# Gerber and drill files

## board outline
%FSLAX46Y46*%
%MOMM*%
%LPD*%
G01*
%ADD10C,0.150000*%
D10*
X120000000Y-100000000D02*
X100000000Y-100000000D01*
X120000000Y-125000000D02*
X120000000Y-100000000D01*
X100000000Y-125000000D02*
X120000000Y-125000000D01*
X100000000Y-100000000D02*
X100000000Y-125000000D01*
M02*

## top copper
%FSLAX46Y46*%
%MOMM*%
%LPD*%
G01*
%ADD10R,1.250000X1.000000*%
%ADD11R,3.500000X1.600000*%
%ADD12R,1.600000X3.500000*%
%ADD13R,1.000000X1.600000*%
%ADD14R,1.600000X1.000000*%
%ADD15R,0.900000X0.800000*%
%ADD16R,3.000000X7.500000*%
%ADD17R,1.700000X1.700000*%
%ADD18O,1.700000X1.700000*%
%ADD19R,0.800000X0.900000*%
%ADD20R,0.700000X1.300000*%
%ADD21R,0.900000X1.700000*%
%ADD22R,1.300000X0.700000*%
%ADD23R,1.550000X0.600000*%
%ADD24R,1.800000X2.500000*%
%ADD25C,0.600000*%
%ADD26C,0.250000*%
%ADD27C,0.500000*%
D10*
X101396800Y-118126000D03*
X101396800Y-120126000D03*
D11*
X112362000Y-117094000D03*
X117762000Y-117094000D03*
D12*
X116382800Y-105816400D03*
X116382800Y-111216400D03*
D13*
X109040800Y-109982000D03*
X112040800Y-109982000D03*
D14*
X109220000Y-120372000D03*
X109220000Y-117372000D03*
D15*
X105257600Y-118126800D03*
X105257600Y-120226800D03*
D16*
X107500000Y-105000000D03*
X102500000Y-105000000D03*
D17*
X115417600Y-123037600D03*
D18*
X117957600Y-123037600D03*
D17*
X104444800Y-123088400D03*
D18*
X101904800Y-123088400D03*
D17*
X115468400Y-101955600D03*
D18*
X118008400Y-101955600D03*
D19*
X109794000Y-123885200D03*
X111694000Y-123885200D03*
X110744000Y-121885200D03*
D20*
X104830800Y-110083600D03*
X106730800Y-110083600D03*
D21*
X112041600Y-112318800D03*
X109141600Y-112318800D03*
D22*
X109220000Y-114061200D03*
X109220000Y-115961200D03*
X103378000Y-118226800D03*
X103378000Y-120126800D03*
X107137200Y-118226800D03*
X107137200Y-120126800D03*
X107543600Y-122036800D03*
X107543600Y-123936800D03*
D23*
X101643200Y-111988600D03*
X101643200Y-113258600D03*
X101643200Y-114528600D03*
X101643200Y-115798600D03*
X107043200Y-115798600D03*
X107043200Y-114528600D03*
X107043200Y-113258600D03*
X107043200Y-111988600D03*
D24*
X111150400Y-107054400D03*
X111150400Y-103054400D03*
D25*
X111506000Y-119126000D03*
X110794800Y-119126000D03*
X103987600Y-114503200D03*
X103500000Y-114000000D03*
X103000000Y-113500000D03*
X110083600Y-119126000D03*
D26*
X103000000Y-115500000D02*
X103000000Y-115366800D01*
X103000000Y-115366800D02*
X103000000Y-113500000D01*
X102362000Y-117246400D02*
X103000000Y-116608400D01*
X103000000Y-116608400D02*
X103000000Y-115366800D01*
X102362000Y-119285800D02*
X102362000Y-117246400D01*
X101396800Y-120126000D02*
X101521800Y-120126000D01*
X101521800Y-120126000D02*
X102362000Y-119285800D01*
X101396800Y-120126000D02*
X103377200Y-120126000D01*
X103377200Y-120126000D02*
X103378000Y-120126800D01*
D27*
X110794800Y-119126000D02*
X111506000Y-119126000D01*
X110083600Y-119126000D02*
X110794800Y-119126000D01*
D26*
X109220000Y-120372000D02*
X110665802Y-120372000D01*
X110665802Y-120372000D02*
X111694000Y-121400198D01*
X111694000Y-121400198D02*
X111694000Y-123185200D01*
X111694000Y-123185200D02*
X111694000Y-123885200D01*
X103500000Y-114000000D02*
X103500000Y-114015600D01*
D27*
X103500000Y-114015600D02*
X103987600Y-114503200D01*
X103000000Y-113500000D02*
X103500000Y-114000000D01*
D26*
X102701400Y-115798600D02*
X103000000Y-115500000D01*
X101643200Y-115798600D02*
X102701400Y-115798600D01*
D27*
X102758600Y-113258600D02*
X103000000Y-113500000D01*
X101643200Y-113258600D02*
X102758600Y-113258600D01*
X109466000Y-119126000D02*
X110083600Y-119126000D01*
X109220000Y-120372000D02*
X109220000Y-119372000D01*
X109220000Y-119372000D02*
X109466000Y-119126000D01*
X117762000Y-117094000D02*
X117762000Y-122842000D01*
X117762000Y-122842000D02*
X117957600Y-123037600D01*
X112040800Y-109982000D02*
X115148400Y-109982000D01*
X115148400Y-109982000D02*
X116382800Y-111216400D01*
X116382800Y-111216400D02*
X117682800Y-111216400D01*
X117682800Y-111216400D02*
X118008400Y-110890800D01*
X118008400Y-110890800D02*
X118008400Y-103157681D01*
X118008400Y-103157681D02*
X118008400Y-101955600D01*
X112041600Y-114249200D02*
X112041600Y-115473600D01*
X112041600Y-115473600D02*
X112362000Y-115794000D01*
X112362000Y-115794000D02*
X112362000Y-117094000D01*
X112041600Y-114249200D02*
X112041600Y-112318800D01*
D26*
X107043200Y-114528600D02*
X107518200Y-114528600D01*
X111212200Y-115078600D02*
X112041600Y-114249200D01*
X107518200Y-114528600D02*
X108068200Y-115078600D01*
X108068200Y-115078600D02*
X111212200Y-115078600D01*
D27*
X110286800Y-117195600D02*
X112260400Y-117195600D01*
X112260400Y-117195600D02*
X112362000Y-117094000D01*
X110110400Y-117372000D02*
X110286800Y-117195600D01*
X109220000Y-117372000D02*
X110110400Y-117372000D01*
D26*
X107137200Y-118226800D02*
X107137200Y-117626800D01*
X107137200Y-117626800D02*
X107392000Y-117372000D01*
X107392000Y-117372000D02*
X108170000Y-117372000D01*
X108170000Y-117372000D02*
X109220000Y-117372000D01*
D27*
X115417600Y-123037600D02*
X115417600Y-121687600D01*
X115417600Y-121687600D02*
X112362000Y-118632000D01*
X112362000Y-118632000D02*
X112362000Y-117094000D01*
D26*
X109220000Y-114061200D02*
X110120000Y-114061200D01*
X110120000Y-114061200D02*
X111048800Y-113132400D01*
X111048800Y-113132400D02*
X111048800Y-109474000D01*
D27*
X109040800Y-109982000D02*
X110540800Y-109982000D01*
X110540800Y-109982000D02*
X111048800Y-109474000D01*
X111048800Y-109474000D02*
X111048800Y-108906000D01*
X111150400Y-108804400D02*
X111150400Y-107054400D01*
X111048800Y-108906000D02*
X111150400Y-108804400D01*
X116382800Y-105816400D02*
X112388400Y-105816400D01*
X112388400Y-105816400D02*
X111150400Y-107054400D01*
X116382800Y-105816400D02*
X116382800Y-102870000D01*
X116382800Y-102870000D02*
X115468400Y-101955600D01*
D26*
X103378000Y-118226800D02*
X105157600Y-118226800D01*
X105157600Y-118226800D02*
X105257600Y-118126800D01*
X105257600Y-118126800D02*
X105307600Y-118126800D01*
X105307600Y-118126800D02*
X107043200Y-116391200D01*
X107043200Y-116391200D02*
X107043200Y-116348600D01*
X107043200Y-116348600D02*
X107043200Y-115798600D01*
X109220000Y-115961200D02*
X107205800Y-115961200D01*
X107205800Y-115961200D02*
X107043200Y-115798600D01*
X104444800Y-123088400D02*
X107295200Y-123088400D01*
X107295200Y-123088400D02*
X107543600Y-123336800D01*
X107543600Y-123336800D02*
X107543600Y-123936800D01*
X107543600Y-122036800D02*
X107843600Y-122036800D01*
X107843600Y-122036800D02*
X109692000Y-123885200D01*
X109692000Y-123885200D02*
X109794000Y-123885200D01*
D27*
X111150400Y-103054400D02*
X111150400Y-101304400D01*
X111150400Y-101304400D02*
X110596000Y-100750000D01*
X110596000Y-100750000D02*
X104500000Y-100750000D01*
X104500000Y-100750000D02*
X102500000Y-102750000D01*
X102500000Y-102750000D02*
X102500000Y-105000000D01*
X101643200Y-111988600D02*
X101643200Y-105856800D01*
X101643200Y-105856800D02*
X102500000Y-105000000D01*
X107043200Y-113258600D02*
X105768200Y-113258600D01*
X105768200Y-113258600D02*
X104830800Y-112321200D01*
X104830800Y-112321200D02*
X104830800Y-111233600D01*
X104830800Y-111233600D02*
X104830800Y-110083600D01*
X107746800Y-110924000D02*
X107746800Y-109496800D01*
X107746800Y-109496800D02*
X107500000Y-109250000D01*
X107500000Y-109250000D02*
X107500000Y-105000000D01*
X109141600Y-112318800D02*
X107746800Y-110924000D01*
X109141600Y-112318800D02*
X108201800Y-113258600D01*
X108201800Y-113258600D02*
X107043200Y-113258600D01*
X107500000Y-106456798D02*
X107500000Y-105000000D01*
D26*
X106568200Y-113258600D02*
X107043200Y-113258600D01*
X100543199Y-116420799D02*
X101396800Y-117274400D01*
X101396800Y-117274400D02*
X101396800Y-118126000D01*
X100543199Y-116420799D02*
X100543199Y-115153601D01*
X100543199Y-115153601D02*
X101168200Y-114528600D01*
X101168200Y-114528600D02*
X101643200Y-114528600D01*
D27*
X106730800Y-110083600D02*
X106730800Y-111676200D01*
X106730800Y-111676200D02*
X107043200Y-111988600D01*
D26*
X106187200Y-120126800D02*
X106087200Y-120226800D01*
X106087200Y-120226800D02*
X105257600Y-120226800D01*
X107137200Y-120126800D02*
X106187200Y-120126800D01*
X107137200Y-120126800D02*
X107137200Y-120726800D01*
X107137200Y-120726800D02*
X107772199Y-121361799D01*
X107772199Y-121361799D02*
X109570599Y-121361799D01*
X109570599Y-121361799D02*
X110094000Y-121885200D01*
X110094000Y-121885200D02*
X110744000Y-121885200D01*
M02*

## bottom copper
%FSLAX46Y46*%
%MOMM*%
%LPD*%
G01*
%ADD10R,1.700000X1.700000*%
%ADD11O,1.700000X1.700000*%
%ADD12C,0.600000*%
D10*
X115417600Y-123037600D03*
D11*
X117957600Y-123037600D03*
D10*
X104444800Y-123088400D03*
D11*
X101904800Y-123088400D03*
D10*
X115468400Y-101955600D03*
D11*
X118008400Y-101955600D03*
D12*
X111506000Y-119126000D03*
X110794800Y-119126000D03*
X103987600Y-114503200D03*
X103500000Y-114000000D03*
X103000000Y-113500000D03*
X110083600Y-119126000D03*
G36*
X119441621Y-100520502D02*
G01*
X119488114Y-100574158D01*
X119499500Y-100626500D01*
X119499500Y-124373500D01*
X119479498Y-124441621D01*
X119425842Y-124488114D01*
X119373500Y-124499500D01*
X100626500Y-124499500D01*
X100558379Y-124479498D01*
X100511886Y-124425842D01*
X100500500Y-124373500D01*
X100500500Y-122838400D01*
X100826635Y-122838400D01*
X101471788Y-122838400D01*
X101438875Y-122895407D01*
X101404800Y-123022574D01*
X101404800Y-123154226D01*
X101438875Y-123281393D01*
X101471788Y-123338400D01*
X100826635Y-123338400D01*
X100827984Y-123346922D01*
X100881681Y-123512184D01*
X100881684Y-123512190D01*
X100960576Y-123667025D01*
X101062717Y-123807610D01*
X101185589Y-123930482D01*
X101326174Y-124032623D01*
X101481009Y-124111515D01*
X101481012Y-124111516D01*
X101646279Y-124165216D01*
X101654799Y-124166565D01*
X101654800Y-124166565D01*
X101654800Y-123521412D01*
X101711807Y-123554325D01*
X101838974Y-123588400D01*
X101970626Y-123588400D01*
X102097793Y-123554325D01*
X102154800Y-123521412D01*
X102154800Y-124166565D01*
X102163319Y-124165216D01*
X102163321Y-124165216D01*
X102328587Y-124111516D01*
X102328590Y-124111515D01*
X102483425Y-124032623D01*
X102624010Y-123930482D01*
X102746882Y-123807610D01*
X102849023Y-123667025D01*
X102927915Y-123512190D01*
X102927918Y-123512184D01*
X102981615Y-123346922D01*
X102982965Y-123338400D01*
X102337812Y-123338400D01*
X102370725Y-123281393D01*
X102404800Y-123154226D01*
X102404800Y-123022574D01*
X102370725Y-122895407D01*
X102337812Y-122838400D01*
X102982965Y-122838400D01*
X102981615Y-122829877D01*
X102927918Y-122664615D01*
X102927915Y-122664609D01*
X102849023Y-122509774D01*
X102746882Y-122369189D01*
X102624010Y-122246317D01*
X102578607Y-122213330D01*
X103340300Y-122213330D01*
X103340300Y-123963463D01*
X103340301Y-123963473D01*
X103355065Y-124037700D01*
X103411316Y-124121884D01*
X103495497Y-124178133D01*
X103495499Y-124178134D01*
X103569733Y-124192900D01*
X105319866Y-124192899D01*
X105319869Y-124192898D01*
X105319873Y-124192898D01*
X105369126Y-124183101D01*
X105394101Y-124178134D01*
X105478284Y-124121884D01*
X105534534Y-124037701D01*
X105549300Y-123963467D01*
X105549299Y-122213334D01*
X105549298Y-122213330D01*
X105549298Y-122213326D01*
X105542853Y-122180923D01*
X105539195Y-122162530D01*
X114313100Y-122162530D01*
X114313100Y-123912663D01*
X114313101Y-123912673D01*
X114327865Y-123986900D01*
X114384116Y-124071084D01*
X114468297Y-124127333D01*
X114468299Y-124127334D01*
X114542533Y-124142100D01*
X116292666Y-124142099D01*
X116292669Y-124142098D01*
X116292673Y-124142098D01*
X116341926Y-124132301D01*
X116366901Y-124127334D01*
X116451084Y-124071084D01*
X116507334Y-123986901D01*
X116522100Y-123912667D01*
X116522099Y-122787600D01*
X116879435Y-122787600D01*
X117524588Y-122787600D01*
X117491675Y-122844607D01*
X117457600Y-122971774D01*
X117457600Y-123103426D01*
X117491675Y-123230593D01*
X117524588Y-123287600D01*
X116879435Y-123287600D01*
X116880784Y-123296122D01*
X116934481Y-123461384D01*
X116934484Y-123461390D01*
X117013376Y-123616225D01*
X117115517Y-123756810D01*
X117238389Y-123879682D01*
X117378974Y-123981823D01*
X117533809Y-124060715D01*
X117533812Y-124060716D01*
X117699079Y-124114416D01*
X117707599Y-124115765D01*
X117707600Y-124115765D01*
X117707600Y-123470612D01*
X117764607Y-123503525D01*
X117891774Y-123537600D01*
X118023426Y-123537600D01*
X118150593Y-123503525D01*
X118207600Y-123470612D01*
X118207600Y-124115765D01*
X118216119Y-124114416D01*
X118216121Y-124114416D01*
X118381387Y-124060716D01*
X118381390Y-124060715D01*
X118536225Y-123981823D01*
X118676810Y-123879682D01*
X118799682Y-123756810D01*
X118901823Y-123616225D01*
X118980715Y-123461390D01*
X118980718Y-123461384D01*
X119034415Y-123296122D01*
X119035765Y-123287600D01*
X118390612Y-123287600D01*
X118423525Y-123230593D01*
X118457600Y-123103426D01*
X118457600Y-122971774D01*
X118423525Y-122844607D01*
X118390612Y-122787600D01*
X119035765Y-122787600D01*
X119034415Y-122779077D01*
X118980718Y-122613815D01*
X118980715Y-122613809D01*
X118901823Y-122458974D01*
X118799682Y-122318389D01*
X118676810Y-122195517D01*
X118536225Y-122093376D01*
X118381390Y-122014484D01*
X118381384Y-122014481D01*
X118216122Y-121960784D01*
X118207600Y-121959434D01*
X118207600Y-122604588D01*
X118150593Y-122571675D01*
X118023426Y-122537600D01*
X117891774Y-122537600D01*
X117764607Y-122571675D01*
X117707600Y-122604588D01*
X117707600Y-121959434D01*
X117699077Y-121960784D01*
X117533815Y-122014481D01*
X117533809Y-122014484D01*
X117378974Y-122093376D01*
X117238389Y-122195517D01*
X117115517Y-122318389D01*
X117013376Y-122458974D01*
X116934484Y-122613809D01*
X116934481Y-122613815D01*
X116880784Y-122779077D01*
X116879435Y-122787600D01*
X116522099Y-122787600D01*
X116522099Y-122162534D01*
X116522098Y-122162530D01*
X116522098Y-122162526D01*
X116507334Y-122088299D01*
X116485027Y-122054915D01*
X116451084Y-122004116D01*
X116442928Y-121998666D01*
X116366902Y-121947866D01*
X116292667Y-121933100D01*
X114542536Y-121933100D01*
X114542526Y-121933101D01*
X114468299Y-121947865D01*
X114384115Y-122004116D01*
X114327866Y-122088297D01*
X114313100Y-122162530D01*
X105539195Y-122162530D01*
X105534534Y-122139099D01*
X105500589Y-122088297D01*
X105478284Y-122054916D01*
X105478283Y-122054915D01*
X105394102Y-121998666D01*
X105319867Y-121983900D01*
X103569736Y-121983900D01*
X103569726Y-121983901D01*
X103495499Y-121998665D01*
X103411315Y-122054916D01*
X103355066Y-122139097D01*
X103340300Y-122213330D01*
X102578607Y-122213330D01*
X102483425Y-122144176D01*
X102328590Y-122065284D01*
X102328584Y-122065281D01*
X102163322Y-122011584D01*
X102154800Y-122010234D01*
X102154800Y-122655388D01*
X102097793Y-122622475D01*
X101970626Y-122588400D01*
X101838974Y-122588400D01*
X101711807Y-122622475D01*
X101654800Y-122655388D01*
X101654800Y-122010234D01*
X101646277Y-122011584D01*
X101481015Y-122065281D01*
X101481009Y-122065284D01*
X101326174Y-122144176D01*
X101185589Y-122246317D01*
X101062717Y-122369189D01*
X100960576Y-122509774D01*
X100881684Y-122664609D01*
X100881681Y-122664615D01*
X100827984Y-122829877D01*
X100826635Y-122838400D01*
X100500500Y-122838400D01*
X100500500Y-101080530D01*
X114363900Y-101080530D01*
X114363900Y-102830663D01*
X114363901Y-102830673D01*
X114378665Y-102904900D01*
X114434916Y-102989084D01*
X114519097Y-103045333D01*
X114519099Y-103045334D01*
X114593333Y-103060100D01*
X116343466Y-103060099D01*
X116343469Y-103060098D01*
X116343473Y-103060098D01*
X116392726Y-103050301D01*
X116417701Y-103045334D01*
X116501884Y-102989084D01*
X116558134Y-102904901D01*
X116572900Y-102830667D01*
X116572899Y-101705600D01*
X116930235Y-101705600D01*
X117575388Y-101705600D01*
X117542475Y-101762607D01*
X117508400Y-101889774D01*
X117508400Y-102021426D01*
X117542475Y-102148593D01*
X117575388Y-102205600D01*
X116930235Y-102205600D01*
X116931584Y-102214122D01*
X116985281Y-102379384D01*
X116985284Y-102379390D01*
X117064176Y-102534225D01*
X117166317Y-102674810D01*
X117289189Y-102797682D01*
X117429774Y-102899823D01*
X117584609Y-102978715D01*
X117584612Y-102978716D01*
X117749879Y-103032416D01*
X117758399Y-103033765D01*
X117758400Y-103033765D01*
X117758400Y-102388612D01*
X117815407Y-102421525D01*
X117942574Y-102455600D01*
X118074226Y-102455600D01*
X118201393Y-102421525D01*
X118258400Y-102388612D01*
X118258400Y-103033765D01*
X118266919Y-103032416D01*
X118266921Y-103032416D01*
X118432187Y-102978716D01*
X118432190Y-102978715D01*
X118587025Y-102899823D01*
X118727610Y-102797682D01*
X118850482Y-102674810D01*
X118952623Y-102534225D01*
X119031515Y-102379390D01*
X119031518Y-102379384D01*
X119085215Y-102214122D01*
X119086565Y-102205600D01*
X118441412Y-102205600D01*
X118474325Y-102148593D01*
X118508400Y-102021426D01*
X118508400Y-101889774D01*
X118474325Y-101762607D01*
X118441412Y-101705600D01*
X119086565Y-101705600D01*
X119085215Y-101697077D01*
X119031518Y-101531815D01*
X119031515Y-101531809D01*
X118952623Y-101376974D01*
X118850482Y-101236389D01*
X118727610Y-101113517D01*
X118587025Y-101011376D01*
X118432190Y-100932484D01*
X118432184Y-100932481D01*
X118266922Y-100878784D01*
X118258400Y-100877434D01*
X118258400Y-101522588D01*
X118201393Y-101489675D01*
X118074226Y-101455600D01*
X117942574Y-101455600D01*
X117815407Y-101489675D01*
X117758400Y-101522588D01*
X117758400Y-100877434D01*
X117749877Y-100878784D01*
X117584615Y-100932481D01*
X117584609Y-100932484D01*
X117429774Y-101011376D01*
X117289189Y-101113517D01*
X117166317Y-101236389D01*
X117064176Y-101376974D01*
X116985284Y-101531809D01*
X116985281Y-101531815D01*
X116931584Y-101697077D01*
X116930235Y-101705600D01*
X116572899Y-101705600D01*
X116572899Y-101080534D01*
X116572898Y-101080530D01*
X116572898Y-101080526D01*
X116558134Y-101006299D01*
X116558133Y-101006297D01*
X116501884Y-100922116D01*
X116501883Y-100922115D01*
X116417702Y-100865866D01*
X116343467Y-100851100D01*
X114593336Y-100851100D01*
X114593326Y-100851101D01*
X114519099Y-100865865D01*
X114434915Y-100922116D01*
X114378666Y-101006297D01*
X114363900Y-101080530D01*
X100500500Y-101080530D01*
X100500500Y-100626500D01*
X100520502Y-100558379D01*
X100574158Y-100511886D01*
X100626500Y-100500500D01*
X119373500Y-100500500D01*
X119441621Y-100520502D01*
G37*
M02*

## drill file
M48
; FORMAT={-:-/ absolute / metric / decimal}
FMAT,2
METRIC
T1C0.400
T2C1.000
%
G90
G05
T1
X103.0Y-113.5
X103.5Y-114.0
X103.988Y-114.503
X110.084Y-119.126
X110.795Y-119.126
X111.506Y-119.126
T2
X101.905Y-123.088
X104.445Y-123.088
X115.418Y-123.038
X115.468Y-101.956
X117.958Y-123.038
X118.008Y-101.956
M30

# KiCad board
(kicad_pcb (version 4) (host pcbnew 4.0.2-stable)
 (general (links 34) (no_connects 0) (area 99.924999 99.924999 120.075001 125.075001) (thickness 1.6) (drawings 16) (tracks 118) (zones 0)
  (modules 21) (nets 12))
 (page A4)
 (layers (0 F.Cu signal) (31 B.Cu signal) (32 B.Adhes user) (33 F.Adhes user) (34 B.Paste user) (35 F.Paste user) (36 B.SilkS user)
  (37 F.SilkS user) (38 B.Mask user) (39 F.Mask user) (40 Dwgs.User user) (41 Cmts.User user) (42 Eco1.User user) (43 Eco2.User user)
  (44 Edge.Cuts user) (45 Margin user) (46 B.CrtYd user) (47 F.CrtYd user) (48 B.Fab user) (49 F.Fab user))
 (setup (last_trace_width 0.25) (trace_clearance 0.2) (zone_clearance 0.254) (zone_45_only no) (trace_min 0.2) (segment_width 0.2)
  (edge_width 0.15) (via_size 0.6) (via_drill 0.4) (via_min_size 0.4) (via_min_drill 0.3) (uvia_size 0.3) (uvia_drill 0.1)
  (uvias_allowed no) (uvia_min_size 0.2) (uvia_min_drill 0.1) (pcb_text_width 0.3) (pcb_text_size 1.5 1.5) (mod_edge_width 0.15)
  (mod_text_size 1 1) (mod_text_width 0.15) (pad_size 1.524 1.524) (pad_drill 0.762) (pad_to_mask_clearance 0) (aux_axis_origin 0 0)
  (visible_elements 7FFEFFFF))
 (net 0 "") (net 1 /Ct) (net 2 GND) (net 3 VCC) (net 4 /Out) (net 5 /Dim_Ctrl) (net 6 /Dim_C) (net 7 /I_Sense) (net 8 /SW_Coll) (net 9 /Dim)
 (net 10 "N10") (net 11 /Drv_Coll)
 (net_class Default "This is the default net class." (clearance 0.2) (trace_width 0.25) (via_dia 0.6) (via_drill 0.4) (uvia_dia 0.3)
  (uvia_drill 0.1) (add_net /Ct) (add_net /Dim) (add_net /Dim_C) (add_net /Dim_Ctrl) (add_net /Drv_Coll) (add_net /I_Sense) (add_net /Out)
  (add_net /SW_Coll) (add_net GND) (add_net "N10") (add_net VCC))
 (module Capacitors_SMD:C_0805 (layer F.Cu) (at 101.3968 119.126 270)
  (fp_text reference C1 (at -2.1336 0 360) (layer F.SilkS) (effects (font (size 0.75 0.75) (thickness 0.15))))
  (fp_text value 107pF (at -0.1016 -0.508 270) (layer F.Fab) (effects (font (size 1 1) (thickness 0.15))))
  (pad 1 smd rect (at -1 0 270) (size 1 1.25) (layers F.Cu F.Paste F.Mask) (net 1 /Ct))
  (pad 2 smd rect (at 1 0 270) (size 1 1.25) (layers F.Cu F.Paste F.Mask) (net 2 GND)))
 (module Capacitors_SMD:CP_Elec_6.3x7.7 (layer F.Cu) (at 115.062 117.094)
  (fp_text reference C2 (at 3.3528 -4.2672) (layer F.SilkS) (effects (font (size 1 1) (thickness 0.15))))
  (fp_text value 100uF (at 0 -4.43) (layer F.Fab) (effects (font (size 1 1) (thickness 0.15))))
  (pad 1 smd rect (at -2.7 0 180) (size 3.5 1.6) (layers F.Cu F.Paste F.Mask) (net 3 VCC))
  (pad 2 smd rect (at 2.7 0 180) (size 3.5 1.6) (layers F.Cu F.Paste F.Mask) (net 2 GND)))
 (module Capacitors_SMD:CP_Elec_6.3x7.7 (layer F.Cu) (at 116.3828 108.5164 270)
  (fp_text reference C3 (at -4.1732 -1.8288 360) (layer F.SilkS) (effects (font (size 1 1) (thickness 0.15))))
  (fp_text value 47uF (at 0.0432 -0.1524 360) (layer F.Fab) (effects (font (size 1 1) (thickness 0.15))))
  (pad 1 smd rect (at -2.7 0 90) (size 3.5 1.6) (layers F.Cu F.Paste F.Mask) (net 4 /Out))
  (pad 2 smd rect (at 2.7 0 90) (size 3.5 1.6) (layers F.Cu F.Paste F.Mask) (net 2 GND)))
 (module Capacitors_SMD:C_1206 (layer F.Cu) (at 110.5408 109.982)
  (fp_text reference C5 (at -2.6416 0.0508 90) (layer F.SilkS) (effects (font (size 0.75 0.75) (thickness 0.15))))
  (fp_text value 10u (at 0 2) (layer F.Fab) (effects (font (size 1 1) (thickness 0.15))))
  (pad 1 smd rect (at -1.5 0) (size 1 1.6) (layers F.Cu F.Paste F.Mask) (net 4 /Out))
  (pad 2 smd rect (at 1.5 0) (size 1 1.6) (layers F.Cu F.Paste F.Mask) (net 2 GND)))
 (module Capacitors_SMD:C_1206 (layer F.Cu) (at 109.22 118.872 90)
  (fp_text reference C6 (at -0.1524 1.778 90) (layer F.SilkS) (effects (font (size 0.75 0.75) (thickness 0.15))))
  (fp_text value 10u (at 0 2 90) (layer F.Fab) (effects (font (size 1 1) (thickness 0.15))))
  (pad 1 smd rect (at -1.5 0 90) (size 1 1.6) (layers F.Cu F.Paste F.Mask) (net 2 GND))
  (pad 2 smd rect (at 1.5 0 90) (size 1 1.6) (layers F.Cu F.Paste F.Mask) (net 3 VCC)))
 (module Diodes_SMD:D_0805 (layer F.Cu) (at 105.2576 119.1768 270)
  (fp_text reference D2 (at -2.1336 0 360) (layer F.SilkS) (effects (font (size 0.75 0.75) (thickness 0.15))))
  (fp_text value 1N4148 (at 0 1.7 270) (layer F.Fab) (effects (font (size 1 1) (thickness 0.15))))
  (pad 1 smd rect (at -1.05 0 270) (size 0.8 0.9) (layers F.Cu F.Paste F.Mask) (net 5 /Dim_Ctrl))
  (pad 2 smd rect (at 1.05 0 270) (size 0.8 0.9) (layers F.Cu F.Paste F.Mask) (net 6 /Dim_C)))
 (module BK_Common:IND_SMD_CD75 (layer F.Cu) (at 105 105 180)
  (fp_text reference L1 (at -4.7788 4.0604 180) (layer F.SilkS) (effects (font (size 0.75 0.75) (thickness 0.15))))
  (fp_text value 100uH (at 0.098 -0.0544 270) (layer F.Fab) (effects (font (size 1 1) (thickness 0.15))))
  (pad 1 smd rect (at -2.5 0 180) (size 3 7.5) (layers F.Cu F.Paste F.Mask) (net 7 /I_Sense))
  (pad 2 smd rect (at 2.5 0 180) (size 3 7.5) (layers F.Cu F.Paste F.Mask) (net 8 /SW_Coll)))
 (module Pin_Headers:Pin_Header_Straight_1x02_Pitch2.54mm (layer F.Cu) (at 115.4176 123.0376 90)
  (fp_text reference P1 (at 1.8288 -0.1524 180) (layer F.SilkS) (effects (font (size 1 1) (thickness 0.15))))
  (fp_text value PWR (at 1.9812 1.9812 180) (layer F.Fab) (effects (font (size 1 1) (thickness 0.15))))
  (pad 1 thru_hole rect (at 0 0 90) (size 1.7 1.7) (drill 1) (layers *.Cu *.Mask) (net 3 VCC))
  (pad 2 thru_hole oval (at 0 2.54 90) (size 1.7 1.7) (drill 1) (layers *.Cu *.Mask) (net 2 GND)))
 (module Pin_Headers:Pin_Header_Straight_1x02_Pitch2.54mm (layer F.Cu) (at 104.4448 123.0884 270)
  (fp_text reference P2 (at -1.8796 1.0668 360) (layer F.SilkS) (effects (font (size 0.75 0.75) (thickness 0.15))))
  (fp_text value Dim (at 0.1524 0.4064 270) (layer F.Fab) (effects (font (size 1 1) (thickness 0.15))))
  (pad 1 thru_hole rect (at 0 0 270) (size 1.7 1.7) (drill 1) (layers *.Cu *.Mask) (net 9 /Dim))
  (pad 2 thru_hole oval (at 0 2.54 270) (size 1.7 1.7) (drill 1) (layers *.Cu *.Mask) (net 2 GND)))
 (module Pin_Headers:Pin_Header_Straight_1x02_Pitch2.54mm (layer F.Cu) (at 115.4684 101.9556 90)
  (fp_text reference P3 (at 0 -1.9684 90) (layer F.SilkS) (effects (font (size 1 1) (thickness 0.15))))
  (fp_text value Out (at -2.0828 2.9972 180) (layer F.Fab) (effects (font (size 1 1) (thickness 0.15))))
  (pad 1 thru_hole rect (at 0 0 90) (size 1.7 1.7) (drill 1) (layers *.Cu *.Mask) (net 4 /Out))
  (pad 2 thru_hole oval (at 0 2.54 90) (size 1.7 1.7) (drill 1) (layers *.Cu *.Mask) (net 2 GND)))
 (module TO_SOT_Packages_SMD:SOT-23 (layer F.Cu) (at 110.744 122.8852 90)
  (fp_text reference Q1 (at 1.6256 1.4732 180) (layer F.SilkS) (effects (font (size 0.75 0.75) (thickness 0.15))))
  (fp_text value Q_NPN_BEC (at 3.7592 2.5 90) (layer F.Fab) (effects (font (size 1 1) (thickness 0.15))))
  (pad 1 smd rect (at -1 -0.95 90) (size 0.9 0.8) (layers F.Cu F.Paste F.Mask) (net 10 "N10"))
  (pad 2 smd rect (at -1 0.95 90) (size 0.9 0.8) (layers F.Cu F.Paste F.Mask) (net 2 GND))
  (pad 3 smd rect (at 1 0 90) (size 0.9 0.8) (layers F.Cu F.Paste F.Mask) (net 6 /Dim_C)))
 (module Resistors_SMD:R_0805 (layer F.Cu) (at 105.7808 110.0836)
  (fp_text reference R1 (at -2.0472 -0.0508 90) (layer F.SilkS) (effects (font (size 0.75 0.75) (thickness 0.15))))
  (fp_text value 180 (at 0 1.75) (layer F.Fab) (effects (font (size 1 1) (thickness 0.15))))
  (pad 1 smd rect (at -0.95 0) (size 0.7 1.3) (layers F.Cu F.Paste F.Mask) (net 7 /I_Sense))
  (pad 2 smd rect (at 0.95 0) (size 0.7 1.3) (layers F.Cu F.Paste F.Mask) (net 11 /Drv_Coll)))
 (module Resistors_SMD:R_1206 (layer F.Cu) (at 110.5916 112.3188 180)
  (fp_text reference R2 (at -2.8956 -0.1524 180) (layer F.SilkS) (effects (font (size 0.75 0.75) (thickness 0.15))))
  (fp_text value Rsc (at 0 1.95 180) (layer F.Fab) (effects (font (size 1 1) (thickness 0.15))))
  (pad 1 smd rect (at -1.45 0 180) (size 0.9 1.7) (layers F.Cu F.Paste F.Mask) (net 3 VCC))
  (pad 2 smd rect (at 1.45 0 180) (size 0.9 1.7) (layers F.Cu F.Paste F.Mask) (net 7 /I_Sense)))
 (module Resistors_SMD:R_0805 (layer F.Cu) (at 109.22 115.0112 270)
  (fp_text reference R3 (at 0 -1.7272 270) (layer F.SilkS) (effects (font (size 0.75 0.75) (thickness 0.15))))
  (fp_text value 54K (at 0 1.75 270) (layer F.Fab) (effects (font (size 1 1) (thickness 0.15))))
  (pad 1 smd rect (at -0.95 0 270) (size 0.7 1.3) (layers F.Cu F.Paste F.Mask) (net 4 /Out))
  (pad 2 smd rect (at 0.95 0 270) (size 0.7 1.3) (layers F.Cu F.Paste F.Mask) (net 5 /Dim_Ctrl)))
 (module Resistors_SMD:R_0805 (layer F.Cu) (at 103.378 119.1768 270)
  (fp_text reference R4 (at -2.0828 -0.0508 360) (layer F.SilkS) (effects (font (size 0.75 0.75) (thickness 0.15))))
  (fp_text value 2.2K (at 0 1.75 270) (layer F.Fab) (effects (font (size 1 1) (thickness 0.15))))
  (pad 1 smd rect (at -0.95 0 270) (size 0.7 1.3) (layers F.Cu F.Paste F.Mask) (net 5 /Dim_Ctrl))
  (pad 2 smd rect (at 0.95 0 270) (size 0.7 1.3) (layers F.Cu F.Paste F.Mask) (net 2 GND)))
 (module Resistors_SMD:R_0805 (layer F.Cu) (at 107.1372 119.1768 270)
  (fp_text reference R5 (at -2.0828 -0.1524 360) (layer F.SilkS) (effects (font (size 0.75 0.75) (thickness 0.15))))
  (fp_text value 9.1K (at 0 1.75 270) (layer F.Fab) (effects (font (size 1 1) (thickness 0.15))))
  (pad 1 smd rect (at -0.95 0 270) (size 0.7 1.3) (layers F.Cu F.Paste F.Mask) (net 3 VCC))
  (pad 2 smd rect (at 0.95 0 270) (size 0.7 1.3) (layers F.Cu F.Paste F.Mask) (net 6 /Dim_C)))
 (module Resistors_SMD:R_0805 (layer F.Cu) (at 107.5436 122.9868 270)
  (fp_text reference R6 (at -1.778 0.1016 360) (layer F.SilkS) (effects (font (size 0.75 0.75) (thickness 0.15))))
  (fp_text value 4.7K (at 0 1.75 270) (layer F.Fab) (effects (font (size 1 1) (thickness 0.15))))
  (pad 1 smd rect (at -0.95 0 270) (size 0.7 1.3) (layers F.Cu F.Paste F.Mask) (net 10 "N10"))
  (pad 2 smd rect (at 0.95 0 270) (size 0.7 1.3) (layers F.Cu F.Paste F.Mask) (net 9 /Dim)))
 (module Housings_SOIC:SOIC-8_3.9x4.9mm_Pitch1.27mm (layer F.Cu) (at 104.3432 113.8936)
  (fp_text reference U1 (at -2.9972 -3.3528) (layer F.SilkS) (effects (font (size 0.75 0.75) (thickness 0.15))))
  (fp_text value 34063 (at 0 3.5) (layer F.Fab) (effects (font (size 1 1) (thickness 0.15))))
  (pad 1 smd rect (at -2.7 -1.905) (size 1.55 0.6) (layers F.Cu F.Paste F.Mask) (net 8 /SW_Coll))
  (pad 2 smd rect (at -2.7 -0.635) (size 1.55 0.6) (layers F.Cu F.Paste F.Mask) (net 2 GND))
  (pad 3 smd rect (at -2.7 0.635) (size 1.55 0.6) (layers F.Cu F.Paste F.Mask) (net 1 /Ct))
  (pad 4 smd rect (at -2.7 1.905) (size 1.55 0.6) (layers F.Cu F.Paste F.Mask) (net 2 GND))
  (pad 5 smd rect (at 2.7 1.905) (size 1.55 0.6) (layers F.Cu F.Paste F.Mask) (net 5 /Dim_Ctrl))
  (pad 6 smd rect (at 2.7 0.635) (size 1.55 0.6) (layers F.Cu F.Paste F.Mask) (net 3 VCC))
  (pad 7 smd rect (at 2.7 -0.635) (size 1.55 0.6) (layers F.Cu F.Paste F.Mask) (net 7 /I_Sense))
  (pad 8 smd rect (at 2.7 -1.905) (size 1.55 0.6) (layers F.Cu F.Paste F.Mask) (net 11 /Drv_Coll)))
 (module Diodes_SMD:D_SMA (layer F.Cu) (at 111.1504 105.0544 90)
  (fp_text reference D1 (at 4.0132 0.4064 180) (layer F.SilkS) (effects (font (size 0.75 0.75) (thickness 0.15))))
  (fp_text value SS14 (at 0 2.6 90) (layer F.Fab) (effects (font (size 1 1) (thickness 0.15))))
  (pad 1 smd rect (at -2 0 90) (size 2.5 1.8) (layers F.Cu F.Paste F.Mask) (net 4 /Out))
  (pad 2 smd rect (at 2 0 90) (size 2.5 1.8) (layers F.Cu F.Paste F.Mask) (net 8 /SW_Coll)))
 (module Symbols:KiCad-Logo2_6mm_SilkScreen (layer B.Cu) (at 109.9312 115 180)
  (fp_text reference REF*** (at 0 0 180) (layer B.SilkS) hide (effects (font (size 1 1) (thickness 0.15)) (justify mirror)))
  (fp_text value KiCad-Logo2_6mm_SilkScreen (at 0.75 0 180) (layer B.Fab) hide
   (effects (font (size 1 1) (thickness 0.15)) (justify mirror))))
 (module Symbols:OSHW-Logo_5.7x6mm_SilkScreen (layer B.Cu) (at 114 108.8 180)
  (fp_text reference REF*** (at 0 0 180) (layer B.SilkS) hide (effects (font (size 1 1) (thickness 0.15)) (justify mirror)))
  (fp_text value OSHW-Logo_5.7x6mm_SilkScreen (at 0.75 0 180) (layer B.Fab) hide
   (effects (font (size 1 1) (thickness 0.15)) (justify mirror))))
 (gr_line (start 120 100) (end 100 100) (layer Edge.Cuts) (width 0.15))
 (gr_line (start 120 125) (end 120 100) (layer Edge.Cuts) (width 0.15))
 (gr_line (start 100 125) (end 120 125) (layer Edge.Cuts) (width 0.15))
 (gr_line (start 100 100) (end 100 125) (layer Edge.Cuts) (width 0.15))
 (segment (start 103 115.5) (end 103 115.3668) (width 0.25) (layer F.Cu) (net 2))
 (segment (start 103 115.3668) (end 103 113.5) (width 0.25) (layer F.Cu) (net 2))
 (segment (start 102.362 117.2464) (end 103 116.6084) (width 0.25) (layer F.Cu) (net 2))
 (segment (start 103 116.6084) (end 103 115.3668) (width 0.25) (layer F.Cu) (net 2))
 (segment (start 102.362 119.2858) (end 102.362 117.2464) (width 0.25) (layer F.Cu) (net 2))
 (segment (start 101.3968 120.126) (end 101.5218 120.126) (width 0.25) (layer F.Cu) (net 2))
 (segment (start 101.5218 120.126) (end 102.362 119.2858) (width 0.25) (layer F.Cu) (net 2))
 (segment (start 101.3968 120.126) (end 103.3772 120.126) (width 0.25) (layer F.Cu) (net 2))
 (segment (start 103.3772 120.126) (end 103.378 120.1268) (width 0.25) (layer F.Cu) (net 2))
 (segment (start 110.7948 119.126) (end 111.506 119.126) (width 0.5) (layer F.Cu) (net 2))
 (via (at 111.506 119.126) (size 0.6) (drill 0.4) (layers F.Cu B.Cu) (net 2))
 (segment (start 110.0836 119.126) (end 110.7948 119.126) (width 0.5) (layer F.Cu) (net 2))
 (via (at 110.7948 119.126) (size 0.6) (drill 0.4) (layers F.Cu B.Cu) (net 2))
 (segment (start 109.22 120.372) (end 110.665802 120.372) (width 0.25) (layer F.Cu) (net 2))
 (segment (start 110.665802 120.372) (end 111.694 121.400198) (width 0.25) (layer F.Cu) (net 2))
 (segment (start 111.694 121.400198) (end 111.694 123.1852) (width 0.25) (layer F.Cu) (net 2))
 (segment (start 111.694 123.1852) (end 111.694 123.8852) (width 0.25) (layer F.Cu) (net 2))
 (segment (start 103.5 114) (end 103.5 114.0156) (width 0.25) (layer F.Cu) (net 2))
 (segment (start 103.5 114.0156) (end 103.9876 114.5032) (width 0.5) (layer F.Cu) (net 2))
 (via (at 103.9876 114.5032) (size 0.6) (drill 0.4) (layers F.Cu B.Cu) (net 2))
 (via (at 103.5 114) (size 0.6) (drill 0.4) (layers F.Cu B.Cu) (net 2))
 (segment (start 103 113.5) (end 103.5 114) (width 0.5) (layer F.Cu) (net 2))
 (segment (start 102.7014 115.7986) (end 103 115.5) (width 0.25) (layer F.Cu) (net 2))
 (segment (start 101.6432 115.7986) (end 102.7014 115.7986) (width 0.25) (layer F.Cu) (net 2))
 (segment (start 102.7586 113.2586) (end 103 113.5) (width 0.5) (layer F.Cu) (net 2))
 (via (at 103 113.5) (size 0.6) (drill 0.4) (layers F.Cu B.Cu) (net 2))
 (segment (start 101.6432 113.2586) (end 102.7586 113.2586) (width 0.5) (layer F.Cu) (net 2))
 (via (at 110.0836 119.126) (size 0.6) (drill 0.4) (layers F.Cu B.Cu) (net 2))
 (segment (start 109.466 119.126) (end 110.0836 119.126) (width 0.5) (layer F.Cu) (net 2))
 (segment (start 109.22 120.372) (end 109.22 119.372) (width 0.5) (layer F.Cu) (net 2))
 (segment (start 109.22 119.372) (end 109.466 119.126) (width 0.5) (layer F.Cu) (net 2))
 (segment (start 117.762 117.094) (end 117.762 122.842) (width 0.5) (layer F.Cu) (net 2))
 (segment (start 117.762 122.842) (end 117.9576 123.0376) (width 0.5) (layer F.Cu) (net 2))
 (segment (start 112.0408 109.982) (end 115.1484 109.982) (width 0.5) (layer F.Cu) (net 2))
 (segment (start 115.1484 109.982) (end 116.3828 111.2164) (width 0.5) (layer F.Cu) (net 2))
 (segment (start 116.3828 111.2164) (end 117.6828 111.2164) (width 0.5) (layer F.Cu) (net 2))
 (segment (start 117.6828 111.2164) (end 118.0084 110.8908) (width 0.5) (layer F.Cu) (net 2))
 (segment (start 118.0084 110.8908) (end 118.0084 103.157681) (width 0.5) (layer F.Cu) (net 2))
 (segment (start 118.0084 103.157681) (end 118.0084 101.9556) (width 0.5) (layer F.Cu) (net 2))
 (segment (start 112.0416 114.2492) (end 112.0416 115.4736) (width 0.5) (layer F.Cu) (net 3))
 (segment (start 112.0416 115.4736) (end 112.362 115.794) (width 0.5) (layer F.Cu) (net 3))
 (segment (start 112.362 115.794) (end 112.362 117.094) (width 0.5) (layer F.Cu) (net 3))
 (segment (start 112.0416 114.2492) (end 112.0416 112.3188) (width 0.5) (layer F.Cu) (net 3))
 (segment (start 107.0432 114.5286) (end 107.5182 114.5286) (width 0.25) (layer F.Cu) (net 3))
 (segment (start 111.2122 115.0786) (end 112.0416 114.2492) (width 0.25) (layer F.Cu) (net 3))
 (segment (start 107.5182 114.5286) (end 108.0682 115.0786) (width 0.25) (layer F.Cu) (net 3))
 (segment (start 108.0682 115.0786) (end 111.2122 115.0786) (width 0.25) (layer F.Cu) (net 3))
 (segment (start 110.2868 117.1956) (end 112.2604 117.1956) (width 0.5) (layer F.Cu) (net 3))
 (segment (start 112.2604 117.1956) (end 112.362 117.094) (width 0.5) (layer F.Cu) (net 3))
 (segment (start 110.1104 117.372) (end 110.2868 117.1956) (width 0.5) (layer F.Cu) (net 3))
 (segment (start 109.22 117.372) (end 110.1104 117.372) (width 0.5) (layer F.Cu) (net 3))
 (segment (start 107.1372 118.2268) (end 107.1372 117.6268) (width 0.25) (layer F.Cu) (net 3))
 (segment (start 107.1372 117.6268) (end 107.392 117.372) (width 0.25) (layer F.Cu) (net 3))
 (segment (start 107.392 117.372) (end 108.17 117.372) (width 0.25) (layer F.Cu) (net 3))
 (segment (start 108.17 117.372) (end 109.22 117.372) (width 0.25) (layer F.Cu) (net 3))
 (segment (start 115.4176 123.0376) (end 115.4176 121.6876) (width 0.5) (layer F.Cu) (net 3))
 (segment (start 115.4176 121.6876) (end 112.362 118.632) (width 0.5) (layer F.Cu) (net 3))
 (segment (start 112.362 118.632) (end 112.362 117.094) (width 0.5) (layer F.Cu) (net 3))
 (segment (start 109.22 114.0612) (end 110.12 114.0612) (width 0.25) (layer F.Cu) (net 4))
 (segment (start 110.12 114.0612) (end 111.0488 113.1324) (width 0.25) (layer F.Cu) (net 4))
 (segment (start 111.0488 113.1324) (end 111.0488 109.474) (width 0.25) (layer F.Cu) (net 4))
 (segment (start 109.0408 109.982) (end 110.5408 109.982) (width 0.5) (layer F.Cu) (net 4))
 (segment (start 110.5408 109.982) (end 111.0488 109.474) (width 0.5) (layer F.Cu) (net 4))
 (segment (start 111.0488 109.474) (end 111.0488 108.906) (width 0.5) (layer F.Cu) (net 4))
 (segment (start 111.1504 108.8044) (end 111.1504 107.0544) (width 0.5) (layer F.Cu) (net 4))
 (segment (start 111.0488 108.906) (end 111.1504 108.8044) (width 0.5) (layer F.Cu) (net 4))
 (segment (start 116.3828 105.8164) (end 112.3884 105.8164) (width 0.5) (layer F.Cu) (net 4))
 (segment (start 112.3884 105.8164) (end 111.1504 107.0544) (width 0.5) (layer F.Cu) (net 4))
 (segment (start 116.3828 105.8164) (end 116.3828 102.87) (width 0.5) (layer F.Cu) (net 4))
 (segment (start 116.3828 102.87) (end 115.4684 101.9556) (width 0.5) (layer F.Cu) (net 4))
 (segment (start 103.378 118.2268) (end 105.1576 118.2268) (width 0.25) (layer F.Cu) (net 5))
 (segment (start 105.1576 118.2268) (end 105.2576 118.1268) (width 0.25) (layer F.Cu) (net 5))
 (segment (start 105.2576 118.1268) (end 105.3076 118.1268) (width 0.25) (layer F.Cu) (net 5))
 (segment (start 105.3076 118.1268) (end 107.0432 116.3912) (width 0.25) (layer F.Cu) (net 5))
 (segment (start 107.0432 116.3912) (end 107.0432 116.3486) (width 0.25) (layer F.Cu) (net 5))
 (segment (start 107.0432 116.3486) (end 107.0432 115.7986) (width 0.25) (layer F.Cu) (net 5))
 (segment (start 109.22 115.9612) (end 107.2058 115.9612) (width 0.25) (layer F.Cu) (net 5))
 (segment (start 107.2058 115.9612) (end 107.0432 115.7986) (width 0.25) (layer F.Cu) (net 5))
 (segment (start 104.4448 123.0884) (end 107.2952 123.0884) (width 0.25) (layer F.Cu) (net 9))
 (segment (start 107.2952 123.0884) (end 107.5436 123.3368) (width 0.25) (layer F.Cu) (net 9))
 (segment (start 107.5436 123.3368) (end 107.5436 123.9368) (width 0.25) (layer F.Cu) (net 9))
 (segment (start 107.5436 122.0368) (end 107.8436 122.0368) (width 0.25) (layer F.Cu) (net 10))
 (segment (start 107.8436 122.0368) (end 109.692 123.8852) (width 0.25) (layer F.Cu) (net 10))
 (segment (start 109.692 123.8852) (end 109.794 123.8852) (width 0.25) (layer F.Cu) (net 10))
 (segment (start 111.1504 103.0544) (end 111.1504 101.3044) (width 0.5) (layer F.Cu) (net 8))
 (segment (start 111.1504 101.3044) (end 110.596 100.75) (width 0.5) (layer F.Cu) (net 8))
 (segment (start 110.596 100.75) (end 104.5 100.75) (width 0.5) (layer F.Cu) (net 8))
 (segment (start 104.5 100.75) (end 102.5 102.75) (width 0.5) (layer F.Cu) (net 8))
 (segment (start 102.5 102.75) (end 102.5 105) (width 0.5) (layer F.Cu) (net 8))
 (segment (start 101.6432 111.9886) (end 101.6432 105.8568) (width 0.5) (layer F.Cu) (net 8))
 (segment (start 101.6432 105.8568) (end 102.5 105) (width 0.5) (layer F.Cu) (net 8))
 (segment (start 107.0432 113.2586) (end 105.7682 113.2586) (width 0.5) (layer F.Cu) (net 7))
 (segment (start 105.7682 113.2586) (end 104.8308 112.3212) (width 0.5) (layer F.Cu) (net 7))
 (segment (start 104.8308 112.3212) (end 104.8308 111.2336) (width 0.5) (layer F.Cu) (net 7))
 (segment (start 104.8308 111.2336) (end 104.8308 110.0836) (width 0.5) (layer F.Cu) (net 7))
 (segment (start 107.7468 110.924) (end 107.7468 109.4968) (width 0.5) (layer F.Cu) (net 7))
 (segment (start 107.7468 109.4968) (end 107.5 109.25) (width 0.5) (layer F.Cu) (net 7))
 (segment (start 107.5 109.25) (end 107.5 105) (width 0.5) (layer F.Cu) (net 7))
 (segment (start 109.1416 112.3188) (end 107.7468 110.924) (width 0.5) (layer F.Cu) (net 7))
 (segment (start 109.1416 112.3188) (end 108.2018 113.2586) (width 0.5) (layer F.Cu) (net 7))
 (segment (start 108.2018 113.2586) (end 107.0432 113.2586) (width 0.5) (layer F.Cu) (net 7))
 (segment (start 107.5 106.456798) (end 107.5 105) (width 0.5) (layer F.Cu) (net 7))
 (segment (start 106.5682 113.2586) (end 107.0432 113.2586) (width 0.25) (layer F.Cu) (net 7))
 (segment (start 100.543199 116.420799) (end 101.3968 117.2744) (width 0.25) (layer F.Cu) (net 1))
 (segment (start 101.3968 117.2744) (end 101.3968 118.126) (width 0.25) (layer F.Cu) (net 1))
 (segment (start 100.543199 116.420799) (end 100.543199 115.153601) (width 0.25) (layer F.Cu) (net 1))
 (segment (start 100.543199 115.153601) (end 101.1682 114.5286) (width 0.25) (layer F.Cu) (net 1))
 (segment (start 101.1682 114.5286) (end 101.6432 114.5286) (width 0.25) (layer F.Cu) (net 1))
 (segment (start 106.7308 110.0836) (end 106.7308 111.6762) (width 0.5) (layer F.Cu) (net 11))
 (segment (start 106.7308 111.6762) (end 107.0432 111.9886) (width 0.5) (layer F.Cu) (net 11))
 (segment (start 106.1872 120.1268) (end 106.0872 120.2268) (width 0.25) (layer F.Cu) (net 6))
 (segment (start 106.0872 120.2268) (end 105.2576 120.2268) (width 0.25) (layer F.Cu) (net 6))
 (segment (start 107.1372 120.1268) (end 106.1872 120.1268) (width 0.25) (layer F.Cu) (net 6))
 (segment (start 107.1372 120.1268) (end 107.1372 120.7268) (width 0.25) (layer F.Cu) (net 6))
 (segment (start 107.1372 120.7268) (end 107.772199 121.361799) (width 0.25) (layer F.Cu) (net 6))
 (segment (start 107.772199 121.361799) (end 109.570599 121.361799) (width 0.25) (layer F.Cu) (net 6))
 (segment (start 109.570599 121.361799) (end 110.094 121.8852) (width 0.25) (layer F.Cu) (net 6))
 (segment (start 110.094 121.8852) (end 110.744 121.8852) (width 0.25) (layer F.Cu) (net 6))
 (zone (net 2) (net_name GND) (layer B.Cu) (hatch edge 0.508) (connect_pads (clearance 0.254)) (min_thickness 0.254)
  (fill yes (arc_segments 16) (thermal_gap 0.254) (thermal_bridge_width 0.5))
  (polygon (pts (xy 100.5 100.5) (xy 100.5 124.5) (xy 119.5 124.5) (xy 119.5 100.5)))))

